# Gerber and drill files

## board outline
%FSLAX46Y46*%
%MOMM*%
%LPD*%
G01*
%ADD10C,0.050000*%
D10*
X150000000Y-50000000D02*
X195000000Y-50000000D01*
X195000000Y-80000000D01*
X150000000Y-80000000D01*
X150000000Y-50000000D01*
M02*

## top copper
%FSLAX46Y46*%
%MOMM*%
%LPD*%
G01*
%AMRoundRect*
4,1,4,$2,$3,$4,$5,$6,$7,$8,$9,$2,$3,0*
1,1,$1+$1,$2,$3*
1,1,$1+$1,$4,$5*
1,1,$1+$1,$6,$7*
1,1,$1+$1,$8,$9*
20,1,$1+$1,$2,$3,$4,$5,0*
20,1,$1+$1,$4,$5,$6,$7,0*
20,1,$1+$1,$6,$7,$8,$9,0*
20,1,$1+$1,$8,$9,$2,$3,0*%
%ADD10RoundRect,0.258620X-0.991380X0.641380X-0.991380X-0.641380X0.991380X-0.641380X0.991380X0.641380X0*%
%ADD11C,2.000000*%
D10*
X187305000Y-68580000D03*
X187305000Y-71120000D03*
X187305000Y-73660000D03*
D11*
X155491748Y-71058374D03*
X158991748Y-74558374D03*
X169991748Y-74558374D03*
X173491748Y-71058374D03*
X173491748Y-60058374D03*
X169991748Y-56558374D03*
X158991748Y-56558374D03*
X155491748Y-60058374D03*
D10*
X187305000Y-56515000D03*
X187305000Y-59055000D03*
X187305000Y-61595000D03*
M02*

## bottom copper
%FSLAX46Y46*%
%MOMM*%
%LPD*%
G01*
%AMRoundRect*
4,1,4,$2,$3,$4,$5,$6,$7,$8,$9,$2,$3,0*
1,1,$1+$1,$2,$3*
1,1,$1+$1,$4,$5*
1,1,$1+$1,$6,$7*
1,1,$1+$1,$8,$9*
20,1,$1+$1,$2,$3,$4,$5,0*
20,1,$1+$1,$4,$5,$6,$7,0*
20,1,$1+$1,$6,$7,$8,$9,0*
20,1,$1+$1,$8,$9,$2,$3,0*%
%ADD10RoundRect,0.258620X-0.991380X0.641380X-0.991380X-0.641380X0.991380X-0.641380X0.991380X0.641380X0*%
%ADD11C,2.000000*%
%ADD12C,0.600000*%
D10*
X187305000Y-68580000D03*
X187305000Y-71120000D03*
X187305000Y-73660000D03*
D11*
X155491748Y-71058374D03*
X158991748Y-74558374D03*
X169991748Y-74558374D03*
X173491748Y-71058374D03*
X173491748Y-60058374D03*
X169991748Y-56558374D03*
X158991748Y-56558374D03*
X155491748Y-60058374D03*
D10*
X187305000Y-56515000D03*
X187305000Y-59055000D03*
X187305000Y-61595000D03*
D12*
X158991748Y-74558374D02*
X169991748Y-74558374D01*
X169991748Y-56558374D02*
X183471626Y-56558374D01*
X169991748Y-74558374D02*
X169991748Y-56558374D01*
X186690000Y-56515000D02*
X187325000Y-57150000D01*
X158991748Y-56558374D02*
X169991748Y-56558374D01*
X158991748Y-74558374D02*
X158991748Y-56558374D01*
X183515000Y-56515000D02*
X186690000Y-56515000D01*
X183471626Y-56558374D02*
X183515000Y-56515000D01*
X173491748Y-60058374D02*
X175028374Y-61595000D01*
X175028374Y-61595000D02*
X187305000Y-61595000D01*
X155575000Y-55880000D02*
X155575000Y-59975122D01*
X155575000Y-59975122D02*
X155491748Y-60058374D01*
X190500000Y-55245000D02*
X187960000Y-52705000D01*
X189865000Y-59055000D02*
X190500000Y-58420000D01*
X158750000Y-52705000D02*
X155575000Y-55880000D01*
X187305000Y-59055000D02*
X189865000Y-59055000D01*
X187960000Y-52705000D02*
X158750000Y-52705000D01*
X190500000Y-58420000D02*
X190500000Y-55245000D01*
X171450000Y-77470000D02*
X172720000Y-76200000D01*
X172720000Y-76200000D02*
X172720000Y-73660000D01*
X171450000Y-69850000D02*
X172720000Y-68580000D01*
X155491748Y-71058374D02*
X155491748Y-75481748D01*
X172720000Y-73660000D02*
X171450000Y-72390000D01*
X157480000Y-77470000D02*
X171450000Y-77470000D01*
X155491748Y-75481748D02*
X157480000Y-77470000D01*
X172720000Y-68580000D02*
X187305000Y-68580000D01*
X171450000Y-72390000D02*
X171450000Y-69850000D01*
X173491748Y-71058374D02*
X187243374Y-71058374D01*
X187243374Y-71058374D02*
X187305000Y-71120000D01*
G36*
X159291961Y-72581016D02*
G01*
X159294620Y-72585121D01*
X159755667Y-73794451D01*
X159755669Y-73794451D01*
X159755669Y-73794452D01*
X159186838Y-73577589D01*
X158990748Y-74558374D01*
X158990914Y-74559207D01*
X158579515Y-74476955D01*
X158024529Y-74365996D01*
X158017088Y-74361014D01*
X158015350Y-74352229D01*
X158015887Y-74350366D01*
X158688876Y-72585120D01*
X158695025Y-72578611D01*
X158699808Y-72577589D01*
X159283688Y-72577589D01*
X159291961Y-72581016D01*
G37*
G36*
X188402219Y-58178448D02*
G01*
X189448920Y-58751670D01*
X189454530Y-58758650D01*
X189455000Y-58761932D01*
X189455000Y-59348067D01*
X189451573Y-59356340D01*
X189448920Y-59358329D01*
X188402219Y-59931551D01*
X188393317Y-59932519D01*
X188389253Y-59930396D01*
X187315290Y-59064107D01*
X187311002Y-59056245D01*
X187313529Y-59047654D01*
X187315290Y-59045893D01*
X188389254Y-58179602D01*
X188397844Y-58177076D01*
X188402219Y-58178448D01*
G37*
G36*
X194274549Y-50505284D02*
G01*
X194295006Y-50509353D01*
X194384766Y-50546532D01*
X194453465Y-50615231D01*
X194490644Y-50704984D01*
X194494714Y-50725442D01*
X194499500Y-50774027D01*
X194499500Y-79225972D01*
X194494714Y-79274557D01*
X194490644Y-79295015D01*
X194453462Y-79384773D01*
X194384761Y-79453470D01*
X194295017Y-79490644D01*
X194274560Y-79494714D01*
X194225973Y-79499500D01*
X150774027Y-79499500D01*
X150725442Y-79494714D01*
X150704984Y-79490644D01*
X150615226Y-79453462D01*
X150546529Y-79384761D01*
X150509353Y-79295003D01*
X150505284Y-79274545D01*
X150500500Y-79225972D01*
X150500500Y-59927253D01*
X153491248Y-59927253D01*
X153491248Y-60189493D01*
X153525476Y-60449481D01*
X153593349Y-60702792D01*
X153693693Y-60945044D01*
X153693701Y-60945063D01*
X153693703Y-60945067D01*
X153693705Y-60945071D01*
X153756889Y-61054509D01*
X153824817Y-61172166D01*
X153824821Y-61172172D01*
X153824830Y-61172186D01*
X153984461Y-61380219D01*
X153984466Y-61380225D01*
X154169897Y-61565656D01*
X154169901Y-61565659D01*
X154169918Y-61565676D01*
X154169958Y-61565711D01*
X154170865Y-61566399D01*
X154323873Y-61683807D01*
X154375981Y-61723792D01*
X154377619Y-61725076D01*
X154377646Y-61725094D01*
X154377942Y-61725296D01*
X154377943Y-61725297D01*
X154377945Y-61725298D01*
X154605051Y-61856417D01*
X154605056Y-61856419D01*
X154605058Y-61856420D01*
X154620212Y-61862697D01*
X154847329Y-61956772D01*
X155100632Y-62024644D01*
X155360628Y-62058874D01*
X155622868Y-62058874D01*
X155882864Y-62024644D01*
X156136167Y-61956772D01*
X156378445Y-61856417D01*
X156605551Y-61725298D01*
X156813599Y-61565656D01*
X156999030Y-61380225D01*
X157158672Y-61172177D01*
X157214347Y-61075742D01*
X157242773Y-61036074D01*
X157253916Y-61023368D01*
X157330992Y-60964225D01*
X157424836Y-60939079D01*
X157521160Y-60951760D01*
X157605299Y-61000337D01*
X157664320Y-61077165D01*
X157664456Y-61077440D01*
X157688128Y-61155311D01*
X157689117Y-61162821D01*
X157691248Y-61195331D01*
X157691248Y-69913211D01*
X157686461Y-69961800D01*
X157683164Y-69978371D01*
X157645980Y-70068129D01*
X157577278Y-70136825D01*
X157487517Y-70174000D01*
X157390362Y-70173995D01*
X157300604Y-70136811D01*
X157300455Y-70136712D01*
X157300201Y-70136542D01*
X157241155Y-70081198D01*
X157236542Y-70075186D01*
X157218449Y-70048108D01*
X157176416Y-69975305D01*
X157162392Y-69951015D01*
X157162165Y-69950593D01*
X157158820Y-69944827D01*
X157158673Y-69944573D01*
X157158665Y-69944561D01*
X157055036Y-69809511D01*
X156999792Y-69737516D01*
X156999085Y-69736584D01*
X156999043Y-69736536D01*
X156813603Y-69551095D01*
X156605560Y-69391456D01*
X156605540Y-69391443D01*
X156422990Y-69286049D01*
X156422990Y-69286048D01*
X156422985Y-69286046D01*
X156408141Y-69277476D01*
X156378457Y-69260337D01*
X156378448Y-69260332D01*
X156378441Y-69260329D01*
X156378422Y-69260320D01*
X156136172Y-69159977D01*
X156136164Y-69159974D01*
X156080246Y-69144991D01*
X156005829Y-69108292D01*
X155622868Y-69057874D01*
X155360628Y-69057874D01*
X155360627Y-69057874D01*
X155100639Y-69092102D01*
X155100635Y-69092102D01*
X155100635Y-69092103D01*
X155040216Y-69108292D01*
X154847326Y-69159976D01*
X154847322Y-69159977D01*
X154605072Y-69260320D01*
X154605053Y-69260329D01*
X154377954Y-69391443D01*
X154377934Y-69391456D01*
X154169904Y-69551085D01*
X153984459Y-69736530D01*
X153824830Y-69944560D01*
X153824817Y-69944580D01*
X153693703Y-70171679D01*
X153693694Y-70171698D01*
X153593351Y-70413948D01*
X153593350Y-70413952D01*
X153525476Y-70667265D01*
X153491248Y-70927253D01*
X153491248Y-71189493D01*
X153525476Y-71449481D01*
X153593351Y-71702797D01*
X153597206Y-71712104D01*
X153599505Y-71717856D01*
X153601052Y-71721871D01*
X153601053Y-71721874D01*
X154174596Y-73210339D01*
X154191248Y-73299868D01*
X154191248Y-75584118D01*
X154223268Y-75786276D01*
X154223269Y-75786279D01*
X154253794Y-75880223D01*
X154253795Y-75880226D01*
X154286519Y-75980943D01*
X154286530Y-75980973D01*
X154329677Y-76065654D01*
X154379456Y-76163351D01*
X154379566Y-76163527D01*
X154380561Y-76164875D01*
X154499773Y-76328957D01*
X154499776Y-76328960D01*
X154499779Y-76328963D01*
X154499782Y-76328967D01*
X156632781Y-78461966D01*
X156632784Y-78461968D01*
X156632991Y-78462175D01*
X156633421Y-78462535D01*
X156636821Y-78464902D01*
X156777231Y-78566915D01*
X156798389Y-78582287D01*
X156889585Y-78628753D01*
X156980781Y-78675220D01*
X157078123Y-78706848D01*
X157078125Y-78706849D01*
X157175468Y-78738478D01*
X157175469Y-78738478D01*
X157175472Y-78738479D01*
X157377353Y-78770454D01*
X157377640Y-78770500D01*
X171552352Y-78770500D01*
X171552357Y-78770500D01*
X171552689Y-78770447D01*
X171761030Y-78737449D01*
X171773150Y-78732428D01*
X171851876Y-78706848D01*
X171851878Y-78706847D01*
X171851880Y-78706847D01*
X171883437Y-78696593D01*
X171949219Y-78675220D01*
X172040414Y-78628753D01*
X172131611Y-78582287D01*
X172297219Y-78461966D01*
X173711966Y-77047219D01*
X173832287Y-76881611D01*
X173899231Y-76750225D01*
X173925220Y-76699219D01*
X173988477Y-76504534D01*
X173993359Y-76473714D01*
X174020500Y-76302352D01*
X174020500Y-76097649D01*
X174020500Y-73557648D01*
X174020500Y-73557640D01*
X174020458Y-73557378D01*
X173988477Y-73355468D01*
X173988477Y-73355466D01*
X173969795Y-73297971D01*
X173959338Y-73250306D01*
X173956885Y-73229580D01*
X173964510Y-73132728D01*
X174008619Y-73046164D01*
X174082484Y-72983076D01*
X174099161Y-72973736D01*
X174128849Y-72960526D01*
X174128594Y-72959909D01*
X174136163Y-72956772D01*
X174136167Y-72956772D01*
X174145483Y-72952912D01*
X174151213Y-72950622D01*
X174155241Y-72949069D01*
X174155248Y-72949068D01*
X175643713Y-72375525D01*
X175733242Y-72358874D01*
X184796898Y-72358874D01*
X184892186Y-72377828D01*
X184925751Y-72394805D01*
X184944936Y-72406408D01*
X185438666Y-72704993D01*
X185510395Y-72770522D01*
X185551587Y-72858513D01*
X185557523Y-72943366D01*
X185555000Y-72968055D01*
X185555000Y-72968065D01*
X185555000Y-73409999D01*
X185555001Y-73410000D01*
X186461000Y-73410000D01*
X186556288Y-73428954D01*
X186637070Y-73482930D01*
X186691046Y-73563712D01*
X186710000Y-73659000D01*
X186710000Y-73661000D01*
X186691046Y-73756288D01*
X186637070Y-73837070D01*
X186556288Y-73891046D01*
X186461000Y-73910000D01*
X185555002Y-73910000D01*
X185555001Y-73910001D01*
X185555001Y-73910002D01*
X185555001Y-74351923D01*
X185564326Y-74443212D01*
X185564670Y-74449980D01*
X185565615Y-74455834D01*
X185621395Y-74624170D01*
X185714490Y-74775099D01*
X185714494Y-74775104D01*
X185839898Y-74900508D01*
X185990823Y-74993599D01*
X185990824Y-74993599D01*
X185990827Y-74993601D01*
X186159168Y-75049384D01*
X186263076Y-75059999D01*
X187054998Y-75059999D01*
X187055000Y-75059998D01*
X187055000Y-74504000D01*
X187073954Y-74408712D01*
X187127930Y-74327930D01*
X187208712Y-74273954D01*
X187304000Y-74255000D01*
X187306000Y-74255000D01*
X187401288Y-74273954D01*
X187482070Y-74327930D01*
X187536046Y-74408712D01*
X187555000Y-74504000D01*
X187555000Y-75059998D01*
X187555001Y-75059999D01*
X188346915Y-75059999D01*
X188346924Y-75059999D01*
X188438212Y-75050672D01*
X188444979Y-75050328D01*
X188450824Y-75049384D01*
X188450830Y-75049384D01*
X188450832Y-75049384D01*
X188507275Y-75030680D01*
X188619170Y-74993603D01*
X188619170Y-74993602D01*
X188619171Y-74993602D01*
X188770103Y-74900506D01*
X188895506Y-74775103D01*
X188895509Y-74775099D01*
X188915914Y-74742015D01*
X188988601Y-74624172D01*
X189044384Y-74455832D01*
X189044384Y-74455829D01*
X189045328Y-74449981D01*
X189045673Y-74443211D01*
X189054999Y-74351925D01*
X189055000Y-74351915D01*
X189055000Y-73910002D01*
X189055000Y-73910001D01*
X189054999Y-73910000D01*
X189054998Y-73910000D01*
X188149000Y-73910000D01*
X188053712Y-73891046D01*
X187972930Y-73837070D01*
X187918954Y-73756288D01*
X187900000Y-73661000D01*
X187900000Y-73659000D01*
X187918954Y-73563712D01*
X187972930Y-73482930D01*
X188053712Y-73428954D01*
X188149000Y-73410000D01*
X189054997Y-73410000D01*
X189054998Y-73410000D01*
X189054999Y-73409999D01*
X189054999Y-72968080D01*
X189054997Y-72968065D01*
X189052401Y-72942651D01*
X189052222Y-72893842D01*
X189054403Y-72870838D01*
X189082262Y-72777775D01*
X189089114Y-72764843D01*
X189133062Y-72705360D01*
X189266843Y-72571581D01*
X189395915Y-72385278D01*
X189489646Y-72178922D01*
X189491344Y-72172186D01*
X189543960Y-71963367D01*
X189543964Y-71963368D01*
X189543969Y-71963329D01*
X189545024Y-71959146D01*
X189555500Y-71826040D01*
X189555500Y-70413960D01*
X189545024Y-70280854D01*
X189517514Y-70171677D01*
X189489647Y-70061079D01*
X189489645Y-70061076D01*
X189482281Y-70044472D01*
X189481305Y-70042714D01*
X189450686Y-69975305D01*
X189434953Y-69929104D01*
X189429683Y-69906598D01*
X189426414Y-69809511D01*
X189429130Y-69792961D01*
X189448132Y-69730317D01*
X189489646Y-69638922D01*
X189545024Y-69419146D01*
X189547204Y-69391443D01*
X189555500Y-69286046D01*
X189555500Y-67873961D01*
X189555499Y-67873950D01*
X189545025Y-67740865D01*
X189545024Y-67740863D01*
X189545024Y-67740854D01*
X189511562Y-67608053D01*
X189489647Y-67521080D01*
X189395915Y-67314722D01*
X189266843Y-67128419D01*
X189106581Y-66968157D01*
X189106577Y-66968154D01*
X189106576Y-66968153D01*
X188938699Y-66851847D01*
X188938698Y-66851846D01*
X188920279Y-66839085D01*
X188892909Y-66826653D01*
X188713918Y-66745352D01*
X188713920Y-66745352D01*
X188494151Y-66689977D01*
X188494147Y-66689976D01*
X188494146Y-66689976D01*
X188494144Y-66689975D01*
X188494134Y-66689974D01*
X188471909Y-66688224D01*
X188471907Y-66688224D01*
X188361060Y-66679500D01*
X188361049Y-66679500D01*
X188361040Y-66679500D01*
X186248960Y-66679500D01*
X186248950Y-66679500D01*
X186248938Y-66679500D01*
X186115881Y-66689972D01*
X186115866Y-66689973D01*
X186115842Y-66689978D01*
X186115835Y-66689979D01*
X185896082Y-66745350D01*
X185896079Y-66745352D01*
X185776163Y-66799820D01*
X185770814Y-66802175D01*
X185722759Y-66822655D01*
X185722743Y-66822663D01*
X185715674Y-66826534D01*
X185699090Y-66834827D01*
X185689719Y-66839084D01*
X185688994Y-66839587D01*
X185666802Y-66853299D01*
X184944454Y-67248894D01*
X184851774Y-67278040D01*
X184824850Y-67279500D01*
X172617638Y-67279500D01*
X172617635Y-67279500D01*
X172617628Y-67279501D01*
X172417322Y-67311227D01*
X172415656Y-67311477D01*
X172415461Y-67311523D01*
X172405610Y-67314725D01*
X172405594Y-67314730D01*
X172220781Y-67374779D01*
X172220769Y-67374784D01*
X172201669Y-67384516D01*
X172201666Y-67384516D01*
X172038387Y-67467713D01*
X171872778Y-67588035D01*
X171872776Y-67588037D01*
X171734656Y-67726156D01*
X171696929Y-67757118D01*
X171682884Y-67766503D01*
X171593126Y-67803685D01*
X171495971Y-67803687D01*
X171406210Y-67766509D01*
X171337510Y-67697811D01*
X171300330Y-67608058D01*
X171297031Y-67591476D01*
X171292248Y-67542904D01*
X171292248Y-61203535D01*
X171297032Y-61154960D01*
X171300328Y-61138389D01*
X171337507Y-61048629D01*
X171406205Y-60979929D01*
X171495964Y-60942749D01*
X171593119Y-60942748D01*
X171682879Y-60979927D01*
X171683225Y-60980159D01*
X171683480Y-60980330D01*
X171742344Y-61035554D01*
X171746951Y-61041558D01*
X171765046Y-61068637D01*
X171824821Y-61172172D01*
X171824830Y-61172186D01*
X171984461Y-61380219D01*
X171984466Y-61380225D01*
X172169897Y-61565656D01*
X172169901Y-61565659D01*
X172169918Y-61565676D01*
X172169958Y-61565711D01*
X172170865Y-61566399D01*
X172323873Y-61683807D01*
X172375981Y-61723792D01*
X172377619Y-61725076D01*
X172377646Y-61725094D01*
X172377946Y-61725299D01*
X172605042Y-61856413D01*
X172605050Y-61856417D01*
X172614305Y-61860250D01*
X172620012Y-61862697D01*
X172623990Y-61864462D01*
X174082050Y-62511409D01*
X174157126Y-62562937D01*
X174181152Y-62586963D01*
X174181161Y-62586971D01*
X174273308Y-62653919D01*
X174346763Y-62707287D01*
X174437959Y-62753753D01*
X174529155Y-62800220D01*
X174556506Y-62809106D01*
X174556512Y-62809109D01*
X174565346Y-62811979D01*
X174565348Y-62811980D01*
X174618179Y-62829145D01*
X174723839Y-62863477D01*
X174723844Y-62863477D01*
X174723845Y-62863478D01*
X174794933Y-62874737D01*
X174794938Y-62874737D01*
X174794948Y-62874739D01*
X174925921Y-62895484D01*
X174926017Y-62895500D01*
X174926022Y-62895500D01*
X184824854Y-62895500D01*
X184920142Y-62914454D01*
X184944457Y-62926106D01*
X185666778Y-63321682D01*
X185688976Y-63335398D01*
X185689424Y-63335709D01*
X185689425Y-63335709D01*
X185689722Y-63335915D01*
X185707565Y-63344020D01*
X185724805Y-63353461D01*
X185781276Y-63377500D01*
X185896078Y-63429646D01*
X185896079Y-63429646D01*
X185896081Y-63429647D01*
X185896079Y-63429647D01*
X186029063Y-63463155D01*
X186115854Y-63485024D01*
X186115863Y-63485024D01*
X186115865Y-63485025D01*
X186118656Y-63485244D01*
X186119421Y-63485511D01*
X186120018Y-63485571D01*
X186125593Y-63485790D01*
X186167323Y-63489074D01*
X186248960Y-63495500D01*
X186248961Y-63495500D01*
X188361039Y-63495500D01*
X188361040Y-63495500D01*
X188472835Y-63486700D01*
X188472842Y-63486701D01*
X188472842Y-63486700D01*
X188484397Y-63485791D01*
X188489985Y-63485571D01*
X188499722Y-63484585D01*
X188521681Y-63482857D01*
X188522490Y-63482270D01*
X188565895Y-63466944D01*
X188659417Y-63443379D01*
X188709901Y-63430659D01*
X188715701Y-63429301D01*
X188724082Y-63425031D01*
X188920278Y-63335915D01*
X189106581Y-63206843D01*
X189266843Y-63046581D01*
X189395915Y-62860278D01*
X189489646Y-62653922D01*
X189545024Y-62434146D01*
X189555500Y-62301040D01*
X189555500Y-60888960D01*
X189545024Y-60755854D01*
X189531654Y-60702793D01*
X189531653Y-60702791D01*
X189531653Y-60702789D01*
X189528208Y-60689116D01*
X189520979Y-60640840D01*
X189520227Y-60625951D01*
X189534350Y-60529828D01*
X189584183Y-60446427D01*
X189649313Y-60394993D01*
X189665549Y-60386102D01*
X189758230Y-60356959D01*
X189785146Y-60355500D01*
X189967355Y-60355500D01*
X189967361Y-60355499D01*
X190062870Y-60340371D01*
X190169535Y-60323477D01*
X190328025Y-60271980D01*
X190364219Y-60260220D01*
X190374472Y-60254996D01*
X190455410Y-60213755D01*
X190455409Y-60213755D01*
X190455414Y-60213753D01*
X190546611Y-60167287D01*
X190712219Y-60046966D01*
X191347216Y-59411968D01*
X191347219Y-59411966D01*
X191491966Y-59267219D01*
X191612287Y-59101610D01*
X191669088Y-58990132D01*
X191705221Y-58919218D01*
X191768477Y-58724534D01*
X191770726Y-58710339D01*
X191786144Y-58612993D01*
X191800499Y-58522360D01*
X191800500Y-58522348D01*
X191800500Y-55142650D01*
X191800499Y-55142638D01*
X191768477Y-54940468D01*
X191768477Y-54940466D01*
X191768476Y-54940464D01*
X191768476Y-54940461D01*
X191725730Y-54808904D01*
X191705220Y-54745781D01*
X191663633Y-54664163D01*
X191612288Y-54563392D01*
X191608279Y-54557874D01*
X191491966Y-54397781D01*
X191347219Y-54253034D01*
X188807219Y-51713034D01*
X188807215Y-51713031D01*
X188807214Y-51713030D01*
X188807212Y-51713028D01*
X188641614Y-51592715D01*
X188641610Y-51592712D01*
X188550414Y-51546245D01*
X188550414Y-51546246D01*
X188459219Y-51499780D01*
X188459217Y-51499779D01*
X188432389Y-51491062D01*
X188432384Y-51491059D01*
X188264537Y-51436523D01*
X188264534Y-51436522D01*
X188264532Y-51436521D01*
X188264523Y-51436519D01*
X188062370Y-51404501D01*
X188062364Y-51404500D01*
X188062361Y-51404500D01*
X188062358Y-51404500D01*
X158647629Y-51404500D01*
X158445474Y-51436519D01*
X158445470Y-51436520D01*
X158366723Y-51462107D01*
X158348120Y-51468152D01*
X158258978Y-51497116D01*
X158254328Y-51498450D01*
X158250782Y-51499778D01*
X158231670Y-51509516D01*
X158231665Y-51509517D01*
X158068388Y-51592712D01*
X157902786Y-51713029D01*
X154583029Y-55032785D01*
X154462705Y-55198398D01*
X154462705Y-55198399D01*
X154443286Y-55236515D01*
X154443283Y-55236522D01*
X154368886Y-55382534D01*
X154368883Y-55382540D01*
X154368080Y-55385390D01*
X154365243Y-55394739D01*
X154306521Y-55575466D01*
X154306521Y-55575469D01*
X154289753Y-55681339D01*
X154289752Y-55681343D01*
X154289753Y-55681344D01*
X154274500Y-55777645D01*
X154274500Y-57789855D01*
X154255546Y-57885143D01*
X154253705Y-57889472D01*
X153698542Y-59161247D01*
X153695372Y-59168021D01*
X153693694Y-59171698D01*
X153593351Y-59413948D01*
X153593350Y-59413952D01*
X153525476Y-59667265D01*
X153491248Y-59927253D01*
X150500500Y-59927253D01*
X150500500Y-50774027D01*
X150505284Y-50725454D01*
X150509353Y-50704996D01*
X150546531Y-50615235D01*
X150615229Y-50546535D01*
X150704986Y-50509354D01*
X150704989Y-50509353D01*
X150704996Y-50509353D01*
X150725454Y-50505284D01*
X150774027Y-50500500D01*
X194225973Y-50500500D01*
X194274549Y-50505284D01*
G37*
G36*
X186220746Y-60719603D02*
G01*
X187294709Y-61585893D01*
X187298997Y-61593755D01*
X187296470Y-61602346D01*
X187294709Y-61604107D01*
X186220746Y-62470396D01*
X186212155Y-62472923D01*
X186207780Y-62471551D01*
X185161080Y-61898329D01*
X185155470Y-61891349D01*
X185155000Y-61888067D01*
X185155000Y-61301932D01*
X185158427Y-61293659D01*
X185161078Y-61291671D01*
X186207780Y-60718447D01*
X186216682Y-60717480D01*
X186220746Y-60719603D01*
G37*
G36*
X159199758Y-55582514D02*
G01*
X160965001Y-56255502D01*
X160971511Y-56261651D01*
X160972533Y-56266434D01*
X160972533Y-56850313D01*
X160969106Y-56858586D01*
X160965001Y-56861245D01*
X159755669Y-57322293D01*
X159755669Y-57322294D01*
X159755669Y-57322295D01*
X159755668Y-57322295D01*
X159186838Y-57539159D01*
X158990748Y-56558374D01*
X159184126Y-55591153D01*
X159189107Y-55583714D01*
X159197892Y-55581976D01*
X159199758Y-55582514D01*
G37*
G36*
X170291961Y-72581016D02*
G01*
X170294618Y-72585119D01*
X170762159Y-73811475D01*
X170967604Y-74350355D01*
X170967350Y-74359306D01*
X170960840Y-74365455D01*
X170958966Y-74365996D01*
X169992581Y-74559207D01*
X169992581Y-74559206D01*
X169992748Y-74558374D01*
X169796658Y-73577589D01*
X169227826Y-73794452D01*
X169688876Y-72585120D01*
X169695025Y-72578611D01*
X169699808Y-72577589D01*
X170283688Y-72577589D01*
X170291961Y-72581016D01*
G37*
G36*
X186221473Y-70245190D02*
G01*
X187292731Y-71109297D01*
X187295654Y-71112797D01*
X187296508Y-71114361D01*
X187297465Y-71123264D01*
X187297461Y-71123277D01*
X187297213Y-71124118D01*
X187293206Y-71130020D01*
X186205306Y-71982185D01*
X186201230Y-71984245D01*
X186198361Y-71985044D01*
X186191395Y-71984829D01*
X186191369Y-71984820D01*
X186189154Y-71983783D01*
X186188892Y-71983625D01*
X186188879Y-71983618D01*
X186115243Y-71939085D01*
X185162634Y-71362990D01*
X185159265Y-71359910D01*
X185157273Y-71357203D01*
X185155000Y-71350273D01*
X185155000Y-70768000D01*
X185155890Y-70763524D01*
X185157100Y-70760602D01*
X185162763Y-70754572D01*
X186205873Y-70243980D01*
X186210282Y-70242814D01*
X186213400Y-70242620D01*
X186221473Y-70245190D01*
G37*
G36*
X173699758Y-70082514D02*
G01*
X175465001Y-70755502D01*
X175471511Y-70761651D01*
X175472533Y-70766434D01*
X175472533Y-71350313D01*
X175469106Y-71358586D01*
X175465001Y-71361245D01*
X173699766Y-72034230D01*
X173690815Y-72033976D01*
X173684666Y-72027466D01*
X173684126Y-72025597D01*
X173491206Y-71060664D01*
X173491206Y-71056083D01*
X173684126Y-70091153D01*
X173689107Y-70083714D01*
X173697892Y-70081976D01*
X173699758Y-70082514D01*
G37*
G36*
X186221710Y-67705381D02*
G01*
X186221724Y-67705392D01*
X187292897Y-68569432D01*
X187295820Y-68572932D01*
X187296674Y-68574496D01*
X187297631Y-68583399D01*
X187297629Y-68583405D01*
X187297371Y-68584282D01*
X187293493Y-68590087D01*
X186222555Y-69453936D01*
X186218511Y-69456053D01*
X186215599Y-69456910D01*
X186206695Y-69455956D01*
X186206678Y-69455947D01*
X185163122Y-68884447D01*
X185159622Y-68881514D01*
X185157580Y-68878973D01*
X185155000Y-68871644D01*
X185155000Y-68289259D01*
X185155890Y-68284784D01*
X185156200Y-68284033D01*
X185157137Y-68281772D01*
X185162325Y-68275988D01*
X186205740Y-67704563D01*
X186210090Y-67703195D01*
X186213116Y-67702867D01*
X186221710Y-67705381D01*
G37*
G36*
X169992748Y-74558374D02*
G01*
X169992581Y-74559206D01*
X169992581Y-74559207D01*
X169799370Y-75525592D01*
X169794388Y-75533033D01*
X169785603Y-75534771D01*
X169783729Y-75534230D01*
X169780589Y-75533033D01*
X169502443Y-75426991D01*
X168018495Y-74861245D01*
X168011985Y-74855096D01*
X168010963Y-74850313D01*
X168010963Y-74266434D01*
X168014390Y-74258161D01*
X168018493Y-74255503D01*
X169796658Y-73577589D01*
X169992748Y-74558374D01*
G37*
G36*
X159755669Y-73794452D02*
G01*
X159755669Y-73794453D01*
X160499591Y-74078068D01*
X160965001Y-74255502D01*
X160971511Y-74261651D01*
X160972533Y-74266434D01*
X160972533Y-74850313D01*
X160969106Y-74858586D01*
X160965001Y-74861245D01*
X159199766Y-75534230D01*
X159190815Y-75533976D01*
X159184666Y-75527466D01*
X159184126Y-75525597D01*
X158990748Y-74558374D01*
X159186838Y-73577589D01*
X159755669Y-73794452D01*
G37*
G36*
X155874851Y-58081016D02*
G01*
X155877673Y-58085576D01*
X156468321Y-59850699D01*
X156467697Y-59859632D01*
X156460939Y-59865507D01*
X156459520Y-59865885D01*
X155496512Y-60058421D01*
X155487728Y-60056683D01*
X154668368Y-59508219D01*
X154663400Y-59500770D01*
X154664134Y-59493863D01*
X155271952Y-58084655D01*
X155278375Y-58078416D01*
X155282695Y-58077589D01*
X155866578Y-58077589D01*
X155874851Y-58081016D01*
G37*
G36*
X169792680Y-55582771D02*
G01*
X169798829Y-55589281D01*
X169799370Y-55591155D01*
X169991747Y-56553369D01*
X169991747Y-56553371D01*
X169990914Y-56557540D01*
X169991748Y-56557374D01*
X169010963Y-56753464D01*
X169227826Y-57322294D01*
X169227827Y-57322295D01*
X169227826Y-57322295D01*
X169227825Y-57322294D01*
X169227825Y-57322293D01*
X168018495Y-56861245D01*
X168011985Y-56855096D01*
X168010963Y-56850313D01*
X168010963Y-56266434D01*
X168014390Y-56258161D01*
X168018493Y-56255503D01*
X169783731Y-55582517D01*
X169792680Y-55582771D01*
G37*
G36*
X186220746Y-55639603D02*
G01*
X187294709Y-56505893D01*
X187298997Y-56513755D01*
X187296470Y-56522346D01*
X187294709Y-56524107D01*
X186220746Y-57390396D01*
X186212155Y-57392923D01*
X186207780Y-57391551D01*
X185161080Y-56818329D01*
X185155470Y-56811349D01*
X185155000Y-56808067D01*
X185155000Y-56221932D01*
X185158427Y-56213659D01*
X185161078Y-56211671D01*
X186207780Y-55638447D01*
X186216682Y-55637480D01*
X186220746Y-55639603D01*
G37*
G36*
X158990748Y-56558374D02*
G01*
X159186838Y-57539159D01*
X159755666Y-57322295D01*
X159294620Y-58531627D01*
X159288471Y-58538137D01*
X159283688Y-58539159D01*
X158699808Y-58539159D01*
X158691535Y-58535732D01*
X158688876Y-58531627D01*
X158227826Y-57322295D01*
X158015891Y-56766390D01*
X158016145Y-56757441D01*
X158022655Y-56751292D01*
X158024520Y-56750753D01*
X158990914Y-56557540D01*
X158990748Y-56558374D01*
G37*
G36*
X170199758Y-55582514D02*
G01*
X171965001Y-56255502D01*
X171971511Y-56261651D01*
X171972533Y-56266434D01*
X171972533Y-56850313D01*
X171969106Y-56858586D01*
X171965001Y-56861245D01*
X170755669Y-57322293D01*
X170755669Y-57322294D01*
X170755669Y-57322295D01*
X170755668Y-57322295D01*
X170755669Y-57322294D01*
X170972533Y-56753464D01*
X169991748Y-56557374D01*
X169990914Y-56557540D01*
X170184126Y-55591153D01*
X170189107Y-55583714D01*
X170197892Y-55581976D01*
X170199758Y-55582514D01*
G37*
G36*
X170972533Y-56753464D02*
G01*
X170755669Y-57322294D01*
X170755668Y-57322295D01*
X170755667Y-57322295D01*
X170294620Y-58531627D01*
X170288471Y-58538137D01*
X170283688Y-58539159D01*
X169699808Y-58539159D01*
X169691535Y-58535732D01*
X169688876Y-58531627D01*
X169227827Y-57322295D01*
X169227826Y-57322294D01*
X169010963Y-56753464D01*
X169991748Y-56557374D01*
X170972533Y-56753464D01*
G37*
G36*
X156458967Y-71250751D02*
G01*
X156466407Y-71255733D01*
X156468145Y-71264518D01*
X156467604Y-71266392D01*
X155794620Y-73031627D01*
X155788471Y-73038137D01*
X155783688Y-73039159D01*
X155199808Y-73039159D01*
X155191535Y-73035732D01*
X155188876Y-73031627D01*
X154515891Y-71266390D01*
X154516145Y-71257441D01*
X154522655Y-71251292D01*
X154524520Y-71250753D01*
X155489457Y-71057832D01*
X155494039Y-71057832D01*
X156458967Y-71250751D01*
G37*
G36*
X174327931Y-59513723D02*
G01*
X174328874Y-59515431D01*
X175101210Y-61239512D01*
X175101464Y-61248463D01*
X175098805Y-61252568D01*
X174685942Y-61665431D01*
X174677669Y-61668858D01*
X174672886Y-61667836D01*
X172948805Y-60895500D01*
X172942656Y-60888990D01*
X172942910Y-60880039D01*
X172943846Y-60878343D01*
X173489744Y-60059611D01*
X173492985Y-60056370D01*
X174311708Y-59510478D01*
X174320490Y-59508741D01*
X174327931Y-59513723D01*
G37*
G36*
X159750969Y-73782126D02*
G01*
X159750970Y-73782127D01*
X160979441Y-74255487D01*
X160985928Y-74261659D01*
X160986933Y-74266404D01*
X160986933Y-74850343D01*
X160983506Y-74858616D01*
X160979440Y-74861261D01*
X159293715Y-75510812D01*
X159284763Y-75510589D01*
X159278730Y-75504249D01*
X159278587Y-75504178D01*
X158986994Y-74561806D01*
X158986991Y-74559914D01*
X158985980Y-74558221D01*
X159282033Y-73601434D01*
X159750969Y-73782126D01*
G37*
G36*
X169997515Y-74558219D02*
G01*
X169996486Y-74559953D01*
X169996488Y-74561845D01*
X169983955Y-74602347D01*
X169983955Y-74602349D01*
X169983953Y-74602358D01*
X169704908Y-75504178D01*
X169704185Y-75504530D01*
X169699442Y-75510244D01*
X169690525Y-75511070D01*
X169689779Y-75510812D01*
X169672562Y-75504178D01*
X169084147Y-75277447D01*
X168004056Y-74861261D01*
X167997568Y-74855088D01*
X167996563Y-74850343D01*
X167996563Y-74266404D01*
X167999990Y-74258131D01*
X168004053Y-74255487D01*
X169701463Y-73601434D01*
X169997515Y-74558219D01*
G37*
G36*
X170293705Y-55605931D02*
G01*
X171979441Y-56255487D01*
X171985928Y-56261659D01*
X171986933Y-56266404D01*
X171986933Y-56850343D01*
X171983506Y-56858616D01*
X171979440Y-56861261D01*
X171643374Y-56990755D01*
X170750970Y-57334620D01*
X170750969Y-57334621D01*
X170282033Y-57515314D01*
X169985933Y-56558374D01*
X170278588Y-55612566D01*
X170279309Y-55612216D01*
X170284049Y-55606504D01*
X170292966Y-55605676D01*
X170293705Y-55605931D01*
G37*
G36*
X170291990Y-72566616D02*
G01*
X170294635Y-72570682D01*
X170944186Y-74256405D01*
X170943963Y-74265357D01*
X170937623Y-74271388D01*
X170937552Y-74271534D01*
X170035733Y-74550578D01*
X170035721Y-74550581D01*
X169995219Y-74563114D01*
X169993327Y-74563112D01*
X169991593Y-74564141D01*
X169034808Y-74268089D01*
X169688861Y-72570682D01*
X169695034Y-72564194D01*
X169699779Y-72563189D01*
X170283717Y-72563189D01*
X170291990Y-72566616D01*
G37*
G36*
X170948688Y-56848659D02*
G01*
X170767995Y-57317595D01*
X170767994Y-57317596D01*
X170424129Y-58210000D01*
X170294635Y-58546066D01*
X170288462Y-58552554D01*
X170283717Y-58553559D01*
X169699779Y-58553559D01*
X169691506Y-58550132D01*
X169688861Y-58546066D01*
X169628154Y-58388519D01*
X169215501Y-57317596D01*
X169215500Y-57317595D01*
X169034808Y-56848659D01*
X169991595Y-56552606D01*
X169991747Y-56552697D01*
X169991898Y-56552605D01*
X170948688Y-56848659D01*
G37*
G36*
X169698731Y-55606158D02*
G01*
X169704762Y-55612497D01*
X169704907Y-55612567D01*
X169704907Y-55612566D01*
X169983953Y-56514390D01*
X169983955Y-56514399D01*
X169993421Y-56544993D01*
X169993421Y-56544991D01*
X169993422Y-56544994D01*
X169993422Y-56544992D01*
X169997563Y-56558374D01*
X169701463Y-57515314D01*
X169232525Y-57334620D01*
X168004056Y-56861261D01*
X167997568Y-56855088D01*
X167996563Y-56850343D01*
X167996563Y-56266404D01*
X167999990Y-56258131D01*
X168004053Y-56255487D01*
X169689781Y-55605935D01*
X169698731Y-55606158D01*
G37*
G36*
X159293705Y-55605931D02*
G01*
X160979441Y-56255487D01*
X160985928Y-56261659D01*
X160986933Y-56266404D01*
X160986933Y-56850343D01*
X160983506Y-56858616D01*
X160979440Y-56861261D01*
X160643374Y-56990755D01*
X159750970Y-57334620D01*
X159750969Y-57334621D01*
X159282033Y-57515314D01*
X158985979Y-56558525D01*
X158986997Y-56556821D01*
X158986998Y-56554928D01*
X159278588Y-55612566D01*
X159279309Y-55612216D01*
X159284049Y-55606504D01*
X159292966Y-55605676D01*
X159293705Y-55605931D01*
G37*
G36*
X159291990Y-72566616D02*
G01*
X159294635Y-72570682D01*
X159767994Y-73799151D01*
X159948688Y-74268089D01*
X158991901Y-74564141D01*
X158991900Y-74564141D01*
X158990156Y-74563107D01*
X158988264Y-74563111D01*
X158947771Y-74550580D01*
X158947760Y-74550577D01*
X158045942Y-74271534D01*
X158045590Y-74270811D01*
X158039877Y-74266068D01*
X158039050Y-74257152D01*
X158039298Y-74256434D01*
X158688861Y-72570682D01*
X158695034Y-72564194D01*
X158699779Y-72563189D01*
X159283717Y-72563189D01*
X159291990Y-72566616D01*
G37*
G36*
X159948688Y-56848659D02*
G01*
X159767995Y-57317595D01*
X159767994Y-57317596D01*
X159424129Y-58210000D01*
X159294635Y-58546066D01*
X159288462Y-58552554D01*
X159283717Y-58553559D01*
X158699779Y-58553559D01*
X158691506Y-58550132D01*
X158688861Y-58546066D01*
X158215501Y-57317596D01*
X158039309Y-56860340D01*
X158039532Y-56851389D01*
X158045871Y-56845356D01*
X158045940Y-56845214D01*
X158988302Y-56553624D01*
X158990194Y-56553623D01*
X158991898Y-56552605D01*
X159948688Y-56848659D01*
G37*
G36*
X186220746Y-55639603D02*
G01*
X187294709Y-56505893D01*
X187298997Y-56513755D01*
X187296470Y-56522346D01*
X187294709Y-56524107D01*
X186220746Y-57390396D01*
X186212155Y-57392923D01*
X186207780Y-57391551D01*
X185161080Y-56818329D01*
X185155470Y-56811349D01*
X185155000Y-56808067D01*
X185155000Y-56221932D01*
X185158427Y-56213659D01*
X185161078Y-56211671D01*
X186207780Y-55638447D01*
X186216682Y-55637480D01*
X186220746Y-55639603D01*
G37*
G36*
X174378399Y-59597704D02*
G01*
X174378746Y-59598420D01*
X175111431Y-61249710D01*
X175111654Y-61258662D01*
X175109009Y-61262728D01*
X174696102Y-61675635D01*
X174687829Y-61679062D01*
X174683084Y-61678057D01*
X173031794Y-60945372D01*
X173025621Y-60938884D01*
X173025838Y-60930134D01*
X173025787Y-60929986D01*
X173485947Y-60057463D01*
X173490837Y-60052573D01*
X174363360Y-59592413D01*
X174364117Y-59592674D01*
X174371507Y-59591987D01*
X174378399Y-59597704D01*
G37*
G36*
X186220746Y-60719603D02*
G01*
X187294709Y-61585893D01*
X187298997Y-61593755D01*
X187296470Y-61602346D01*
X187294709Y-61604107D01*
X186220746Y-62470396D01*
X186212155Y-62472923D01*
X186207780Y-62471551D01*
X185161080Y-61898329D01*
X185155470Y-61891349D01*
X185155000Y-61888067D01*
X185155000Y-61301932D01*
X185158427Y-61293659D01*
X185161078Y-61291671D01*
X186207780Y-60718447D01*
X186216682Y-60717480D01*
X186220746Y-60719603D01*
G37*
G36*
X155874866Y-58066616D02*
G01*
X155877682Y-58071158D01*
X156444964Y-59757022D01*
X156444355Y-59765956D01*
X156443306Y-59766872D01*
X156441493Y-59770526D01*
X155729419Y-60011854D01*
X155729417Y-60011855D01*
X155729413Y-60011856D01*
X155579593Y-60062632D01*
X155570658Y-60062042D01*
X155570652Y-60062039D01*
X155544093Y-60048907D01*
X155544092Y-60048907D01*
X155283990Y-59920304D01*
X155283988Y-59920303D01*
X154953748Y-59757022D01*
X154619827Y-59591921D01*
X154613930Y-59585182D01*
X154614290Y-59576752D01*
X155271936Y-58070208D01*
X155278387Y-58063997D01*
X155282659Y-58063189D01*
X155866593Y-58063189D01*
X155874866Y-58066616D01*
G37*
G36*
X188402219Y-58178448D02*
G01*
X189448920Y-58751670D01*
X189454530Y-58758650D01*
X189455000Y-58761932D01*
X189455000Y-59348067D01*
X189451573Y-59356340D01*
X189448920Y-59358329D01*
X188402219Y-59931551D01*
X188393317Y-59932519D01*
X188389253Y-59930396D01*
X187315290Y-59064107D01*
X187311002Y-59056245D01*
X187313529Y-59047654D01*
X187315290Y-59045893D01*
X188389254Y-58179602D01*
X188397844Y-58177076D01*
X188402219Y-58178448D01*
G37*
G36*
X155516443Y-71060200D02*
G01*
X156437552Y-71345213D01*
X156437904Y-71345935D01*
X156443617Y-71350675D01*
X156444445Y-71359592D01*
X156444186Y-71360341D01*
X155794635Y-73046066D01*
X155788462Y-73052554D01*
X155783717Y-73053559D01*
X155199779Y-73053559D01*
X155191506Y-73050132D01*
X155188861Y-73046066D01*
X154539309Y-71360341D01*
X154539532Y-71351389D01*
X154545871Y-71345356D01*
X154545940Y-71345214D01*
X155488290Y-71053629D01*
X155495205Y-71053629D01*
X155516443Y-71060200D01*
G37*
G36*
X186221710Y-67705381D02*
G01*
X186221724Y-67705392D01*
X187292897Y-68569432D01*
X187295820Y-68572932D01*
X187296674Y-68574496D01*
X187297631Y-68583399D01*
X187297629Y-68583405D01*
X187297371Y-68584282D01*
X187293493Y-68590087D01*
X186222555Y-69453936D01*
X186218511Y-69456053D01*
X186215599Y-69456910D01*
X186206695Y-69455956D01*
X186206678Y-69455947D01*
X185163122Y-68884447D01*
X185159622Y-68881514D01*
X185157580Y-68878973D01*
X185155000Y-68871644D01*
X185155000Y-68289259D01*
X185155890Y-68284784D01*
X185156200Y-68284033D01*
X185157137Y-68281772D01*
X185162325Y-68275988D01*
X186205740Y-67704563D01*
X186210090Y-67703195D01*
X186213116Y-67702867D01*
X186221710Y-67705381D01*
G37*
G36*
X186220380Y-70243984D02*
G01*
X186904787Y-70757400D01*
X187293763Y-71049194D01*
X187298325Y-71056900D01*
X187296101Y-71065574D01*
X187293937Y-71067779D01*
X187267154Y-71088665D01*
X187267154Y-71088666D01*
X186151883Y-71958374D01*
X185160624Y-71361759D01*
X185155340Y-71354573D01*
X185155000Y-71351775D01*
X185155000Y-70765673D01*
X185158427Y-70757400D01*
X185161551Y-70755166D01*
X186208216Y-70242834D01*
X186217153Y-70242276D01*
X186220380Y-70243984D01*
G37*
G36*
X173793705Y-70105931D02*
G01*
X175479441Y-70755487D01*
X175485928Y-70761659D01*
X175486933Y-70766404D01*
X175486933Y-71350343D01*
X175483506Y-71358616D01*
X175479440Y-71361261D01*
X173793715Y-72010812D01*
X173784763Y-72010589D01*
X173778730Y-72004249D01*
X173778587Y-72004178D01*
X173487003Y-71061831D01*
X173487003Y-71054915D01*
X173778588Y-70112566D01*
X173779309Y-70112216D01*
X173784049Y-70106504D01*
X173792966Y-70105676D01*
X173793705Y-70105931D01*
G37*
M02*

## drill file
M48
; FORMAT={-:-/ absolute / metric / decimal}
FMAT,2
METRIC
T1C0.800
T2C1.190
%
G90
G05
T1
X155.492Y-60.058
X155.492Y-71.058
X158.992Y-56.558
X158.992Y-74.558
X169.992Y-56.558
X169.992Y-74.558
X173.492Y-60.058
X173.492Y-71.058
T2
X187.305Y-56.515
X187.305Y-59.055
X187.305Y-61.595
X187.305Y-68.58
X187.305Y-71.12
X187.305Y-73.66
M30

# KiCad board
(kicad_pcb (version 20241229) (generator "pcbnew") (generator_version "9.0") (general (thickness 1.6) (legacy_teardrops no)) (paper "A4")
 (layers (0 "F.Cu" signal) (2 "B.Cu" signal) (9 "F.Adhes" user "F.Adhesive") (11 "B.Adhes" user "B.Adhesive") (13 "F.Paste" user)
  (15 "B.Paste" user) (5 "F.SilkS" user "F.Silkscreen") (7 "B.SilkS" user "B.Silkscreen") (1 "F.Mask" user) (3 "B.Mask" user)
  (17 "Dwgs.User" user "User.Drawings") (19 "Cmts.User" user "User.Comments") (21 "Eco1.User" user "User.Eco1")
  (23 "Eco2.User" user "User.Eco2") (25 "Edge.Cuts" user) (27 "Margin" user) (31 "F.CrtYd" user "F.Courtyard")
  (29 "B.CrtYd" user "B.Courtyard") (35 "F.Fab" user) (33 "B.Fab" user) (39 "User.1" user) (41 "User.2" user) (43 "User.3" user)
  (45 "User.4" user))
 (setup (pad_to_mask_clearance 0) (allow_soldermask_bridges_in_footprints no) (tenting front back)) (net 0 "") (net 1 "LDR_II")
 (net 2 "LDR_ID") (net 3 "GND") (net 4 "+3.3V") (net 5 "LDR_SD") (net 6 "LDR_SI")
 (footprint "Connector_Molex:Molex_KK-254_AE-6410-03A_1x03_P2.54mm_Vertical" (layer "F.Cu") (at 187.305 68.58 -90)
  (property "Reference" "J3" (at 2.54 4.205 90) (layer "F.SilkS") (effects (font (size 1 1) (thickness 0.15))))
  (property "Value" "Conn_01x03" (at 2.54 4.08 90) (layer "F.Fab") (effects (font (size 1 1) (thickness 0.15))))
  (pad "1" thru_hole roundrect (at 0 0 270) (size 1.8 2.5) (drill 1.19) (layers "*.Cu" "*.Mask") (remove_unused_layers no)
   (roundrect_rratio 0.143678) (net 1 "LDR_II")
   (teardrops (best_length_ratio 0.5) (max_length 1) (best_width_ratio 1) (max_width 2) (curved_edges no) (filter_ratio 0.9) (enabled yes)
    (allow_two_segments yes) (prefer_zone_connections yes)))
  (pad "2" thru_hole roundrect (at 2.54 0 270) (size 1.8 2.5) (drill 1.19) (layers "*.Cu" "*.Mask") (remove_unused_layers no)
   (roundrect_rratio 0.143678) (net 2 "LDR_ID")
   (teardrops (best_length_ratio 0.5) (max_length 1) (best_width_ratio 1) (max_width 2) (curved_edges no) (filter_ratio 0.9) (enabled yes)
    (allow_two_segments yes) (prefer_zone_connections yes)))
  (pad "3" thru_hole roundrect (at 5.08 0 270) (size 1.8 2.5) (drill 1.19) (layers "*.Cu" "*.Mask") (remove_unused_layers no)
   (roundrect_rratio 0.143678) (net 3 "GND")
   (teardrops (best_length_ratio 0.5) (max_length 1) (best_width_ratio 1) (max_width 2) (curved_edges no) (filter_ratio 0.9) (enabled yes)
    (allow_two_segments yes) (prefer_zone_connections yes))))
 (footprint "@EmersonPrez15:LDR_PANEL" (layer "F.Cu") (at 164.991748 65.558374)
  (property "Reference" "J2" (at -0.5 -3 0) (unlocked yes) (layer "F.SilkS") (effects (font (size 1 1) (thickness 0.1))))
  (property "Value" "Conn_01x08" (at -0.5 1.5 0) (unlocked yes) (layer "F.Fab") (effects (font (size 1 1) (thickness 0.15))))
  (pad "1" thru_hole circle (at -9.5 5.5 180) (size 2 2) (drill 0.8) (layers "*.Cu" "*.Mask") (remove_unused_layers no) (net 1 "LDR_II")
   (teardrops (best_length_ratio 0.5) (max_length 1) (best_width_ratio 1) (max_width 2) (curved_edges no) (filter_ratio 0.9) (enabled yes)
    (allow_two_segments yes) (prefer_zone_connections yes)))
  (pad "2" thru_hole circle (at -6 9 90) (size 2 2) (drill 0.8) (layers "*.Cu" "*.Mask") (remove_unused_layers no) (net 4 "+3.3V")
   (teardrops (best_length_ratio 0.5) (max_length 1) (best_width_ratio 1) (max_width 2) (curved_edges no) (filter_ratio 0.9) (enabled yes)
    (allow_two_segments yes) (prefer_zone_connections yes)))
  (pad "3" thru_hole circle (at 5 9 90) (size 2 2) (drill 0.8) (layers "*.Cu" "*.Mask") (remove_unused_layers no) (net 4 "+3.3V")
   (teardrops (best_length_ratio 0.5) (max_length 1) (best_width_ratio 1) (max_width 2) (curved_edges no) (filter_ratio 0.9) (enabled yes)
    (allow_two_segments yes) (prefer_zone_connections yes)))
  (pad "4" thru_hole circle (at 8.5 5.5 180) (size 2 2) (drill 0.8) (layers "*.Cu" "*.Mask") (remove_unused_layers no) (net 2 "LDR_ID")
   (teardrops (best_length_ratio 0.5) (max_length 1) (best_width_ratio 1) (max_width 2) (curved_edges no) (filter_ratio 0.9) (enabled yes)
    (allow_two_segments yes) (prefer_zone_connections yes)))
  (pad "5" thru_hole circle (at 8.5 -5.5 180) (size 2 2) (drill 0.8) (layers "*.Cu" "*.Mask") (remove_unused_layers no) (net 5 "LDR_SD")
   (teardrops (best_length_ratio 0.5) (max_length 1) (best_width_ratio 1) (max_width 2) (curved_edges no) (filter_ratio 0.9) (enabled yes)
    (allow_two_segments yes) (prefer_zone_connections yes)))
  (pad "6" thru_hole circle (at 5 -9 90) (size 2 2) (drill 0.8) (layers "*.Cu" "*.Mask") (remove_unused_layers no) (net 4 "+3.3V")
   (teardrops (best_length_ratio 0.5) (max_length 1) (best_width_ratio 1) (max_width 2) (curved_edges no) (filter_ratio 0.9) (enabled yes)
    (allow_two_segments yes) (prefer_zone_connections yes)))
  (pad "7" thru_hole circle (at -6 -9 90) (size 2 2) (drill 0.8) (layers "*.Cu" "*.Mask") (remove_unused_layers no) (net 4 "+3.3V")
   (teardrops (best_length_ratio 0.5) (max_length 1) (best_width_ratio 1) (max_width 2) (curved_edges no) (filter_ratio 0.9) (enabled yes)
    (allow_two_segments yes) (prefer_zone_connections yes)))
  (pad "8" thru_hole circle (at -9.5 -5.5 180) (size 2 2) (drill 0.8) (layers "*.Cu" "*.Mask") (remove_unused_layers no) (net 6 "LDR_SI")
   (teardrops (best_length_ratio 0.5) (max_length 1) (best_width_ratio 1) (max_width 2) (curved_edges no) (filter_ratio 0.9) (enabled yes)
    (allow_two_segments yes) (prefer_zone_connections yes))))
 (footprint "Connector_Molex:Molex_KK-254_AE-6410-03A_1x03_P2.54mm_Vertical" (layer "F.Cu") (at 187.305 56.515 -90)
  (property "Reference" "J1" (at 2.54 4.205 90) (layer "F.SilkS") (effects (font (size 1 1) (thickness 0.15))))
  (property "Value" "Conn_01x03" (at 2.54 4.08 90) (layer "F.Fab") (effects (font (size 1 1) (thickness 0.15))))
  (pad "1" thru_hole roundrect (at 0 0 270) (size 1.8 2.5) (drill 1.19) (layers "*.Cu" "*.Mask") (remove_unused_layers no)
   (roundrect_rratio 0.143678) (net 4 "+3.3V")
   (teardrops (best_length_ratio 0.5) (max_length 1) (best_width_ratio 1) (max_width 2) (curved_edges no) (filter_ratio 0.9) (enabled yes)
    (allow_two_segments yes) (prefer_zone_connections yes)))
  (pad "2" thru_hole roundrect (at 2.54 0 270) (size 1.8 2.5) (drill 1.19) (layers "*.Cu" "*.Mask") (remove_unused_layers no)
   (roundrect_rratio 0.143678) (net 6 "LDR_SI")
   (teardrops (best_length_ratio 0.5) (max_length 1) (best_width_ratio 1) (max_width 2) (curved_edges no) (filter_ratio 0.9) (enabled yes)
    (allow_two_segments yes) (prefer_zone_connections yes)))
  (pad "3" thru_hole roundrect (at 5.08 0 270) (size 1.8 2.5) (drill 1.19) (layers "*.Cu" "*.Mask") (remove_unused_layers no)
   (roundrect_rratio 0.143678) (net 5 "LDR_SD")
   (teardrops (best_length_ratio 0.5) (max_length 1) (best_width_ratio 1) (max_width 2) (curved_edges no) (filter_ratio 0.9) (enabled yes)
    (allow_two_segments yes) (prefer_zone_connections yes))))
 (gr_rect (start 150 50) (end 195 80) (stroke (width 0.05) (type default)) (fill no) (layer "Edge.Cuts"))
 (segment (start 158.991748 74.558374) (end 169.991748 74.558374) (width 0.6) (layer "B.Cu") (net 4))
 (segment (start 169.991748 56.558374) (end 183.471626 56.558374) (width 0.6) (layer "B.Cu") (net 4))
 (segment (start 169.991748 74.558374) (end 169.991748 56.558374) (width 0.6) (layer "B.Cu") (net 4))
 (segment (start 186.69 56.515) (end 187.325 57.15) (width 0.6) (layer "B.Cu") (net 4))
 (segment (start 158.991748 56.558374) (end 169.991748 56.558374) (width 0.6) (layer "B.Cu") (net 4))
 (segment (start 158.991748 74.558374) (end 158.991748 56.558374) (width 0.6) (layer "B.Cu") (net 4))
 (segment (start 183.515 56.515) (end 186.69 56.515) (width 0.6) (layer "B.Cu") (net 4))
 (segment (start 183.471626 56.558374) (end 183.515 56.515) (width 0.6) (layer "B.Cu") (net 4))
 (segment (start 173.491748 60.058374) (end 175.028374 61.595) (width 0.6) (layer "B.Cu") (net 5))
 (segment (start 175.028374 61.595) (end 187.305 61.595) (width 0.6) (layer "B.Cu") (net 5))
 (segment (start 155.575 55.88) (end 155.575 59.975122) (width 0.6) (layer "B.Cu") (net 6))
 (segment (start 155.575 59.975122) (end 155.491748 60.058374) (width 0.6) (layer "B.Cu") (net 6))
 (segment (start 190.5 55.245) (end 187.96 52.705) (width 0.6) (layer "B.Cu") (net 6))
 (segment (start 189.865 59.055) (end 190.5 58.42) (width 0.6) (layer "B.Cu") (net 6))
 (segment (start 158.75 52.705) (end 155.575 55.88) (width 0.6) (layer "B.Cu") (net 6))
 (segment (start 187.305 59.055) (end 189.865 59.055) (width 0.6) (layer "B.Cu") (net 6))
 (segment (start 187.96 52.705) (end 158.75 52.705) (width 0.6) (layer "B.Cu") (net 6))
 (segment (start 190.5 58.42) (end 190.5 55.245) (width 0.6) (layer "B.Cu") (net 6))
 (segment (start 171.45 77.47) (end 172.72 76.2) (width 0.6) (layer "B.Cu") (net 1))
 (segment (start 172.72 76.2) (end 172.72 73.66) (width 0.6) (layer "B.Cu") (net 1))
 (segment (start 171.45 69.85) (end 172.72 68.58) (width 0.6) (layer "B.Cu") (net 1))
 (segment (start 155.491748 71.058374) (end 155.491748 75.481748) (width 0.6) (layer "B.Cu") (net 1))
 (segment (start 172.72 73.66) (end 171.45 72.39) (width 0.6) (layer "B.Cu") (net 1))
 (segment (start 157.48 77.47) (end 171.45 77.47) (width 0.6) (layer "B.Cu") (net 1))
 (segment (start 155.491748 75.481748) (end 157.48 77.47) (width 0.6) (layer "B.Cu") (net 1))
 (segment (start 172.72 68.58) (end 187.305 68.58) (width 0.6) (layer "B.Cu") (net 1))
 (segment (start 171.45 72.39) (end 171.45 69.85) (width 0.6) (layer "B.Cu") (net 1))
 (segment (start 173.491748 71.058374) (end 187.243374 71.058374) (width 0.6) (layer "B.Cu") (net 2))
 (segment (start 187.243374 71.058374) (end 187.305 71.12) (width 0.6) (layer "B.Cu") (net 2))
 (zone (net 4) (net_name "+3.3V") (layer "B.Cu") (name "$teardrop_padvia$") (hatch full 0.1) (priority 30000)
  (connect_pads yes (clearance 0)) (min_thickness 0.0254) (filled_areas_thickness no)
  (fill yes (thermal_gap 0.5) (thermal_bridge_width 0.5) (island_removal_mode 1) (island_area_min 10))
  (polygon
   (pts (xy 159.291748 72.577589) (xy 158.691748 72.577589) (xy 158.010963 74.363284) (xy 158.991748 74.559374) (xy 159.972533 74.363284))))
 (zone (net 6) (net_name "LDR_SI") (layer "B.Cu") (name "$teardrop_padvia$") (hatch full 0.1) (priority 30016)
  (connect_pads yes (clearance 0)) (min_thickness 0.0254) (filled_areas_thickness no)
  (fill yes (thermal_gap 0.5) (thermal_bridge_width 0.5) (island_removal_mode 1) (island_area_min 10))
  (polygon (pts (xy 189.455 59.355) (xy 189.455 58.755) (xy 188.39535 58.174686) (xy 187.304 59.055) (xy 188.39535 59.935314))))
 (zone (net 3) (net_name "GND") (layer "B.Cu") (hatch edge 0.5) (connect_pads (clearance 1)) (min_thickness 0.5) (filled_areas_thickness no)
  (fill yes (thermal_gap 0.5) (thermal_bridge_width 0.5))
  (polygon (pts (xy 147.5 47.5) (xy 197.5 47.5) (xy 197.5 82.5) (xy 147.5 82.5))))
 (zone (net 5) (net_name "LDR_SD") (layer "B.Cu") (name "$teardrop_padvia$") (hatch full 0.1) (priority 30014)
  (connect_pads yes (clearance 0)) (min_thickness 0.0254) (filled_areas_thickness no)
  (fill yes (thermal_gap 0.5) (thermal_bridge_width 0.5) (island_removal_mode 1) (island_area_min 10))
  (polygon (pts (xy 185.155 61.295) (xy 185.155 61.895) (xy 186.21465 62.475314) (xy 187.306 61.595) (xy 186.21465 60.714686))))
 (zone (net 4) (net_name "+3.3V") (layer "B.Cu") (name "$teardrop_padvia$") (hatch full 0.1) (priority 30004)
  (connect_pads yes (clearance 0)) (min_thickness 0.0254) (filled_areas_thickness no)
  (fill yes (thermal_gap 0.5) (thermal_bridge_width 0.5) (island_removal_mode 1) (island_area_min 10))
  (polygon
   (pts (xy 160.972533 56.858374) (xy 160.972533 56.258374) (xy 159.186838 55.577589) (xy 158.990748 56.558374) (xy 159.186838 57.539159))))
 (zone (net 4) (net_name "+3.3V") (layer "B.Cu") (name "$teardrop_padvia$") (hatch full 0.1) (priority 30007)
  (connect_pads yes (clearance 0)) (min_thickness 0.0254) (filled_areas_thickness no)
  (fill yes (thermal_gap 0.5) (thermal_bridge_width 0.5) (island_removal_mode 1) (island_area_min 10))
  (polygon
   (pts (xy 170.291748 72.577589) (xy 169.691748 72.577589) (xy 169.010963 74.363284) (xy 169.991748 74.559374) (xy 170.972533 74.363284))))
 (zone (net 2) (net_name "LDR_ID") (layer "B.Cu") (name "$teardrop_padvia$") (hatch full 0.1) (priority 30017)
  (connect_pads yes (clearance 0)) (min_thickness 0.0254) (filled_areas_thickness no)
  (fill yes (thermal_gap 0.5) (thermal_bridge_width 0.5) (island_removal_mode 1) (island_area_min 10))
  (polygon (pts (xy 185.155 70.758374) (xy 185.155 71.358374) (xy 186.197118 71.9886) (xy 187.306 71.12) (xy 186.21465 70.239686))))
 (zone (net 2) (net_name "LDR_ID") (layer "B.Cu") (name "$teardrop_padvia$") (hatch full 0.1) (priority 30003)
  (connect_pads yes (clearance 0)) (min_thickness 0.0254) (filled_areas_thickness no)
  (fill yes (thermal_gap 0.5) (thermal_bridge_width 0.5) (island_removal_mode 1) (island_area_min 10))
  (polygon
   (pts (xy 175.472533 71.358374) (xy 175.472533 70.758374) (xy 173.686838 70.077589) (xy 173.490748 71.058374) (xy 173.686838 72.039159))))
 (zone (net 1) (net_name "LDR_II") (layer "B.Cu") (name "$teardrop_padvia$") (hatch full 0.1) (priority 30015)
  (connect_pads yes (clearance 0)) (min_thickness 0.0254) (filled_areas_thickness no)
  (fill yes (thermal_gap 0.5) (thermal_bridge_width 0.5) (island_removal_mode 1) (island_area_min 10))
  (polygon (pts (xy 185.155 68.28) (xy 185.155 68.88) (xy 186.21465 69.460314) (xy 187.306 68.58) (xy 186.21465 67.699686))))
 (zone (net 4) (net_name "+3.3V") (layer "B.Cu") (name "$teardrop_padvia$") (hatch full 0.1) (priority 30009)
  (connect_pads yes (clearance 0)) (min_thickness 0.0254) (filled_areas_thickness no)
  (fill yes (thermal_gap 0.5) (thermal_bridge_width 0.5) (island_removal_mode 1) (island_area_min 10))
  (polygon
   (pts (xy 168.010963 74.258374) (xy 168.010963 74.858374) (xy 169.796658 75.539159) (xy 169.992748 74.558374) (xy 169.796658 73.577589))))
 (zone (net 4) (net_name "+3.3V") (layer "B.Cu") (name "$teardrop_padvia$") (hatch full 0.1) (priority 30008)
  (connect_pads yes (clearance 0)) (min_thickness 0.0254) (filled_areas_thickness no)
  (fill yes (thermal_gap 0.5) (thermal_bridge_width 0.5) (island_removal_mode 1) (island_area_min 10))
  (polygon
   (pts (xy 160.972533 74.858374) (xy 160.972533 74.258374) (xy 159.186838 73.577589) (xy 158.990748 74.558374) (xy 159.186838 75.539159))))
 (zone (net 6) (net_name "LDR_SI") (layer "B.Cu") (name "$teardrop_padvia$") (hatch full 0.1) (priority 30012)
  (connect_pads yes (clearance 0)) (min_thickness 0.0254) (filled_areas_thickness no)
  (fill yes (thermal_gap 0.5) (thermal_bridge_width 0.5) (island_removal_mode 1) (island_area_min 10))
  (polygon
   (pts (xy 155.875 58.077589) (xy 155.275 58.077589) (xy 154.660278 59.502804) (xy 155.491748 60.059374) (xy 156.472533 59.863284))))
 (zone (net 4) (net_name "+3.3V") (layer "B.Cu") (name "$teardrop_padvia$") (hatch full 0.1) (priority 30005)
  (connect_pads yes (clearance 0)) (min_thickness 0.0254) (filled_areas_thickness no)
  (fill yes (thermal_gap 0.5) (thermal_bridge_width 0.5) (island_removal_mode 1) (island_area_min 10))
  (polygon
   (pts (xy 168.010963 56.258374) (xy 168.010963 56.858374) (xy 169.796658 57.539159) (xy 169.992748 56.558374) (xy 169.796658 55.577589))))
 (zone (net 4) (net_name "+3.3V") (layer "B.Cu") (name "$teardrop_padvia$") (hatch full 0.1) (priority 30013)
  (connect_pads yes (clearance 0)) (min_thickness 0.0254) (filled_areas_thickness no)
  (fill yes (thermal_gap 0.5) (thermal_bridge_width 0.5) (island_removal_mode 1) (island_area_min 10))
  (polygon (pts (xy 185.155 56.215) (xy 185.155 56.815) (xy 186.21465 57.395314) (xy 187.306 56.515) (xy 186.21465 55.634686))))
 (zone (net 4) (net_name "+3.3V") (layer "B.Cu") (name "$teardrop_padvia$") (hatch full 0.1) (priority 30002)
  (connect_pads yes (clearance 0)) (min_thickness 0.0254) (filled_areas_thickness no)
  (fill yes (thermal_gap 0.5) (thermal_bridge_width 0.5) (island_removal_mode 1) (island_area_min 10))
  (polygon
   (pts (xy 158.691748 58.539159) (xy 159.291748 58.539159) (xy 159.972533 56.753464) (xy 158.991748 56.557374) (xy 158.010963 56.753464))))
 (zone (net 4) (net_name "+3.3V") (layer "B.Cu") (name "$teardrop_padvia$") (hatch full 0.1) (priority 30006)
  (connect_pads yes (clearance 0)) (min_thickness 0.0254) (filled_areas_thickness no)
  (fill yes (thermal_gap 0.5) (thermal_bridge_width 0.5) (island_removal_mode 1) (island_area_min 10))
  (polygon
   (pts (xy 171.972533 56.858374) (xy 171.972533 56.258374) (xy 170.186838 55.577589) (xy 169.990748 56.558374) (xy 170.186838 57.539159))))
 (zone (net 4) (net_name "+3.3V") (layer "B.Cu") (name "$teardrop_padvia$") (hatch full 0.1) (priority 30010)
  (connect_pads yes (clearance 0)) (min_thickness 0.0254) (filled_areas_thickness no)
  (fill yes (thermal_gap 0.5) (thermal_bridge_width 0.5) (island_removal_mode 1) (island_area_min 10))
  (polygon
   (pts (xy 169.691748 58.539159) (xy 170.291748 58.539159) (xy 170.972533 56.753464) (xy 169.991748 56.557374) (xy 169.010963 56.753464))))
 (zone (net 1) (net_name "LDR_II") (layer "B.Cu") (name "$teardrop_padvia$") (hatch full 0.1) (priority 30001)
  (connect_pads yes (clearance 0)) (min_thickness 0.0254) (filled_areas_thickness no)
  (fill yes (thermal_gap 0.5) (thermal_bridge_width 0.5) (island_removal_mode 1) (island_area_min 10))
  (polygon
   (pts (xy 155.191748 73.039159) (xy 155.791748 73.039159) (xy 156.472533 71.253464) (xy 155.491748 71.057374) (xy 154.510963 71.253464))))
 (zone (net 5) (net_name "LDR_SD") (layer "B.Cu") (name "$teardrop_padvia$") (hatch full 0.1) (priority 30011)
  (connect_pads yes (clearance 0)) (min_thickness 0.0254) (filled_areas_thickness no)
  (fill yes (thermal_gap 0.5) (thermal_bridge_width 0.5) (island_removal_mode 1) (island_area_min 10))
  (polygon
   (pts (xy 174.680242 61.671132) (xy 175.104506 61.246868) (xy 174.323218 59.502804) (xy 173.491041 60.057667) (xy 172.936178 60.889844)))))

